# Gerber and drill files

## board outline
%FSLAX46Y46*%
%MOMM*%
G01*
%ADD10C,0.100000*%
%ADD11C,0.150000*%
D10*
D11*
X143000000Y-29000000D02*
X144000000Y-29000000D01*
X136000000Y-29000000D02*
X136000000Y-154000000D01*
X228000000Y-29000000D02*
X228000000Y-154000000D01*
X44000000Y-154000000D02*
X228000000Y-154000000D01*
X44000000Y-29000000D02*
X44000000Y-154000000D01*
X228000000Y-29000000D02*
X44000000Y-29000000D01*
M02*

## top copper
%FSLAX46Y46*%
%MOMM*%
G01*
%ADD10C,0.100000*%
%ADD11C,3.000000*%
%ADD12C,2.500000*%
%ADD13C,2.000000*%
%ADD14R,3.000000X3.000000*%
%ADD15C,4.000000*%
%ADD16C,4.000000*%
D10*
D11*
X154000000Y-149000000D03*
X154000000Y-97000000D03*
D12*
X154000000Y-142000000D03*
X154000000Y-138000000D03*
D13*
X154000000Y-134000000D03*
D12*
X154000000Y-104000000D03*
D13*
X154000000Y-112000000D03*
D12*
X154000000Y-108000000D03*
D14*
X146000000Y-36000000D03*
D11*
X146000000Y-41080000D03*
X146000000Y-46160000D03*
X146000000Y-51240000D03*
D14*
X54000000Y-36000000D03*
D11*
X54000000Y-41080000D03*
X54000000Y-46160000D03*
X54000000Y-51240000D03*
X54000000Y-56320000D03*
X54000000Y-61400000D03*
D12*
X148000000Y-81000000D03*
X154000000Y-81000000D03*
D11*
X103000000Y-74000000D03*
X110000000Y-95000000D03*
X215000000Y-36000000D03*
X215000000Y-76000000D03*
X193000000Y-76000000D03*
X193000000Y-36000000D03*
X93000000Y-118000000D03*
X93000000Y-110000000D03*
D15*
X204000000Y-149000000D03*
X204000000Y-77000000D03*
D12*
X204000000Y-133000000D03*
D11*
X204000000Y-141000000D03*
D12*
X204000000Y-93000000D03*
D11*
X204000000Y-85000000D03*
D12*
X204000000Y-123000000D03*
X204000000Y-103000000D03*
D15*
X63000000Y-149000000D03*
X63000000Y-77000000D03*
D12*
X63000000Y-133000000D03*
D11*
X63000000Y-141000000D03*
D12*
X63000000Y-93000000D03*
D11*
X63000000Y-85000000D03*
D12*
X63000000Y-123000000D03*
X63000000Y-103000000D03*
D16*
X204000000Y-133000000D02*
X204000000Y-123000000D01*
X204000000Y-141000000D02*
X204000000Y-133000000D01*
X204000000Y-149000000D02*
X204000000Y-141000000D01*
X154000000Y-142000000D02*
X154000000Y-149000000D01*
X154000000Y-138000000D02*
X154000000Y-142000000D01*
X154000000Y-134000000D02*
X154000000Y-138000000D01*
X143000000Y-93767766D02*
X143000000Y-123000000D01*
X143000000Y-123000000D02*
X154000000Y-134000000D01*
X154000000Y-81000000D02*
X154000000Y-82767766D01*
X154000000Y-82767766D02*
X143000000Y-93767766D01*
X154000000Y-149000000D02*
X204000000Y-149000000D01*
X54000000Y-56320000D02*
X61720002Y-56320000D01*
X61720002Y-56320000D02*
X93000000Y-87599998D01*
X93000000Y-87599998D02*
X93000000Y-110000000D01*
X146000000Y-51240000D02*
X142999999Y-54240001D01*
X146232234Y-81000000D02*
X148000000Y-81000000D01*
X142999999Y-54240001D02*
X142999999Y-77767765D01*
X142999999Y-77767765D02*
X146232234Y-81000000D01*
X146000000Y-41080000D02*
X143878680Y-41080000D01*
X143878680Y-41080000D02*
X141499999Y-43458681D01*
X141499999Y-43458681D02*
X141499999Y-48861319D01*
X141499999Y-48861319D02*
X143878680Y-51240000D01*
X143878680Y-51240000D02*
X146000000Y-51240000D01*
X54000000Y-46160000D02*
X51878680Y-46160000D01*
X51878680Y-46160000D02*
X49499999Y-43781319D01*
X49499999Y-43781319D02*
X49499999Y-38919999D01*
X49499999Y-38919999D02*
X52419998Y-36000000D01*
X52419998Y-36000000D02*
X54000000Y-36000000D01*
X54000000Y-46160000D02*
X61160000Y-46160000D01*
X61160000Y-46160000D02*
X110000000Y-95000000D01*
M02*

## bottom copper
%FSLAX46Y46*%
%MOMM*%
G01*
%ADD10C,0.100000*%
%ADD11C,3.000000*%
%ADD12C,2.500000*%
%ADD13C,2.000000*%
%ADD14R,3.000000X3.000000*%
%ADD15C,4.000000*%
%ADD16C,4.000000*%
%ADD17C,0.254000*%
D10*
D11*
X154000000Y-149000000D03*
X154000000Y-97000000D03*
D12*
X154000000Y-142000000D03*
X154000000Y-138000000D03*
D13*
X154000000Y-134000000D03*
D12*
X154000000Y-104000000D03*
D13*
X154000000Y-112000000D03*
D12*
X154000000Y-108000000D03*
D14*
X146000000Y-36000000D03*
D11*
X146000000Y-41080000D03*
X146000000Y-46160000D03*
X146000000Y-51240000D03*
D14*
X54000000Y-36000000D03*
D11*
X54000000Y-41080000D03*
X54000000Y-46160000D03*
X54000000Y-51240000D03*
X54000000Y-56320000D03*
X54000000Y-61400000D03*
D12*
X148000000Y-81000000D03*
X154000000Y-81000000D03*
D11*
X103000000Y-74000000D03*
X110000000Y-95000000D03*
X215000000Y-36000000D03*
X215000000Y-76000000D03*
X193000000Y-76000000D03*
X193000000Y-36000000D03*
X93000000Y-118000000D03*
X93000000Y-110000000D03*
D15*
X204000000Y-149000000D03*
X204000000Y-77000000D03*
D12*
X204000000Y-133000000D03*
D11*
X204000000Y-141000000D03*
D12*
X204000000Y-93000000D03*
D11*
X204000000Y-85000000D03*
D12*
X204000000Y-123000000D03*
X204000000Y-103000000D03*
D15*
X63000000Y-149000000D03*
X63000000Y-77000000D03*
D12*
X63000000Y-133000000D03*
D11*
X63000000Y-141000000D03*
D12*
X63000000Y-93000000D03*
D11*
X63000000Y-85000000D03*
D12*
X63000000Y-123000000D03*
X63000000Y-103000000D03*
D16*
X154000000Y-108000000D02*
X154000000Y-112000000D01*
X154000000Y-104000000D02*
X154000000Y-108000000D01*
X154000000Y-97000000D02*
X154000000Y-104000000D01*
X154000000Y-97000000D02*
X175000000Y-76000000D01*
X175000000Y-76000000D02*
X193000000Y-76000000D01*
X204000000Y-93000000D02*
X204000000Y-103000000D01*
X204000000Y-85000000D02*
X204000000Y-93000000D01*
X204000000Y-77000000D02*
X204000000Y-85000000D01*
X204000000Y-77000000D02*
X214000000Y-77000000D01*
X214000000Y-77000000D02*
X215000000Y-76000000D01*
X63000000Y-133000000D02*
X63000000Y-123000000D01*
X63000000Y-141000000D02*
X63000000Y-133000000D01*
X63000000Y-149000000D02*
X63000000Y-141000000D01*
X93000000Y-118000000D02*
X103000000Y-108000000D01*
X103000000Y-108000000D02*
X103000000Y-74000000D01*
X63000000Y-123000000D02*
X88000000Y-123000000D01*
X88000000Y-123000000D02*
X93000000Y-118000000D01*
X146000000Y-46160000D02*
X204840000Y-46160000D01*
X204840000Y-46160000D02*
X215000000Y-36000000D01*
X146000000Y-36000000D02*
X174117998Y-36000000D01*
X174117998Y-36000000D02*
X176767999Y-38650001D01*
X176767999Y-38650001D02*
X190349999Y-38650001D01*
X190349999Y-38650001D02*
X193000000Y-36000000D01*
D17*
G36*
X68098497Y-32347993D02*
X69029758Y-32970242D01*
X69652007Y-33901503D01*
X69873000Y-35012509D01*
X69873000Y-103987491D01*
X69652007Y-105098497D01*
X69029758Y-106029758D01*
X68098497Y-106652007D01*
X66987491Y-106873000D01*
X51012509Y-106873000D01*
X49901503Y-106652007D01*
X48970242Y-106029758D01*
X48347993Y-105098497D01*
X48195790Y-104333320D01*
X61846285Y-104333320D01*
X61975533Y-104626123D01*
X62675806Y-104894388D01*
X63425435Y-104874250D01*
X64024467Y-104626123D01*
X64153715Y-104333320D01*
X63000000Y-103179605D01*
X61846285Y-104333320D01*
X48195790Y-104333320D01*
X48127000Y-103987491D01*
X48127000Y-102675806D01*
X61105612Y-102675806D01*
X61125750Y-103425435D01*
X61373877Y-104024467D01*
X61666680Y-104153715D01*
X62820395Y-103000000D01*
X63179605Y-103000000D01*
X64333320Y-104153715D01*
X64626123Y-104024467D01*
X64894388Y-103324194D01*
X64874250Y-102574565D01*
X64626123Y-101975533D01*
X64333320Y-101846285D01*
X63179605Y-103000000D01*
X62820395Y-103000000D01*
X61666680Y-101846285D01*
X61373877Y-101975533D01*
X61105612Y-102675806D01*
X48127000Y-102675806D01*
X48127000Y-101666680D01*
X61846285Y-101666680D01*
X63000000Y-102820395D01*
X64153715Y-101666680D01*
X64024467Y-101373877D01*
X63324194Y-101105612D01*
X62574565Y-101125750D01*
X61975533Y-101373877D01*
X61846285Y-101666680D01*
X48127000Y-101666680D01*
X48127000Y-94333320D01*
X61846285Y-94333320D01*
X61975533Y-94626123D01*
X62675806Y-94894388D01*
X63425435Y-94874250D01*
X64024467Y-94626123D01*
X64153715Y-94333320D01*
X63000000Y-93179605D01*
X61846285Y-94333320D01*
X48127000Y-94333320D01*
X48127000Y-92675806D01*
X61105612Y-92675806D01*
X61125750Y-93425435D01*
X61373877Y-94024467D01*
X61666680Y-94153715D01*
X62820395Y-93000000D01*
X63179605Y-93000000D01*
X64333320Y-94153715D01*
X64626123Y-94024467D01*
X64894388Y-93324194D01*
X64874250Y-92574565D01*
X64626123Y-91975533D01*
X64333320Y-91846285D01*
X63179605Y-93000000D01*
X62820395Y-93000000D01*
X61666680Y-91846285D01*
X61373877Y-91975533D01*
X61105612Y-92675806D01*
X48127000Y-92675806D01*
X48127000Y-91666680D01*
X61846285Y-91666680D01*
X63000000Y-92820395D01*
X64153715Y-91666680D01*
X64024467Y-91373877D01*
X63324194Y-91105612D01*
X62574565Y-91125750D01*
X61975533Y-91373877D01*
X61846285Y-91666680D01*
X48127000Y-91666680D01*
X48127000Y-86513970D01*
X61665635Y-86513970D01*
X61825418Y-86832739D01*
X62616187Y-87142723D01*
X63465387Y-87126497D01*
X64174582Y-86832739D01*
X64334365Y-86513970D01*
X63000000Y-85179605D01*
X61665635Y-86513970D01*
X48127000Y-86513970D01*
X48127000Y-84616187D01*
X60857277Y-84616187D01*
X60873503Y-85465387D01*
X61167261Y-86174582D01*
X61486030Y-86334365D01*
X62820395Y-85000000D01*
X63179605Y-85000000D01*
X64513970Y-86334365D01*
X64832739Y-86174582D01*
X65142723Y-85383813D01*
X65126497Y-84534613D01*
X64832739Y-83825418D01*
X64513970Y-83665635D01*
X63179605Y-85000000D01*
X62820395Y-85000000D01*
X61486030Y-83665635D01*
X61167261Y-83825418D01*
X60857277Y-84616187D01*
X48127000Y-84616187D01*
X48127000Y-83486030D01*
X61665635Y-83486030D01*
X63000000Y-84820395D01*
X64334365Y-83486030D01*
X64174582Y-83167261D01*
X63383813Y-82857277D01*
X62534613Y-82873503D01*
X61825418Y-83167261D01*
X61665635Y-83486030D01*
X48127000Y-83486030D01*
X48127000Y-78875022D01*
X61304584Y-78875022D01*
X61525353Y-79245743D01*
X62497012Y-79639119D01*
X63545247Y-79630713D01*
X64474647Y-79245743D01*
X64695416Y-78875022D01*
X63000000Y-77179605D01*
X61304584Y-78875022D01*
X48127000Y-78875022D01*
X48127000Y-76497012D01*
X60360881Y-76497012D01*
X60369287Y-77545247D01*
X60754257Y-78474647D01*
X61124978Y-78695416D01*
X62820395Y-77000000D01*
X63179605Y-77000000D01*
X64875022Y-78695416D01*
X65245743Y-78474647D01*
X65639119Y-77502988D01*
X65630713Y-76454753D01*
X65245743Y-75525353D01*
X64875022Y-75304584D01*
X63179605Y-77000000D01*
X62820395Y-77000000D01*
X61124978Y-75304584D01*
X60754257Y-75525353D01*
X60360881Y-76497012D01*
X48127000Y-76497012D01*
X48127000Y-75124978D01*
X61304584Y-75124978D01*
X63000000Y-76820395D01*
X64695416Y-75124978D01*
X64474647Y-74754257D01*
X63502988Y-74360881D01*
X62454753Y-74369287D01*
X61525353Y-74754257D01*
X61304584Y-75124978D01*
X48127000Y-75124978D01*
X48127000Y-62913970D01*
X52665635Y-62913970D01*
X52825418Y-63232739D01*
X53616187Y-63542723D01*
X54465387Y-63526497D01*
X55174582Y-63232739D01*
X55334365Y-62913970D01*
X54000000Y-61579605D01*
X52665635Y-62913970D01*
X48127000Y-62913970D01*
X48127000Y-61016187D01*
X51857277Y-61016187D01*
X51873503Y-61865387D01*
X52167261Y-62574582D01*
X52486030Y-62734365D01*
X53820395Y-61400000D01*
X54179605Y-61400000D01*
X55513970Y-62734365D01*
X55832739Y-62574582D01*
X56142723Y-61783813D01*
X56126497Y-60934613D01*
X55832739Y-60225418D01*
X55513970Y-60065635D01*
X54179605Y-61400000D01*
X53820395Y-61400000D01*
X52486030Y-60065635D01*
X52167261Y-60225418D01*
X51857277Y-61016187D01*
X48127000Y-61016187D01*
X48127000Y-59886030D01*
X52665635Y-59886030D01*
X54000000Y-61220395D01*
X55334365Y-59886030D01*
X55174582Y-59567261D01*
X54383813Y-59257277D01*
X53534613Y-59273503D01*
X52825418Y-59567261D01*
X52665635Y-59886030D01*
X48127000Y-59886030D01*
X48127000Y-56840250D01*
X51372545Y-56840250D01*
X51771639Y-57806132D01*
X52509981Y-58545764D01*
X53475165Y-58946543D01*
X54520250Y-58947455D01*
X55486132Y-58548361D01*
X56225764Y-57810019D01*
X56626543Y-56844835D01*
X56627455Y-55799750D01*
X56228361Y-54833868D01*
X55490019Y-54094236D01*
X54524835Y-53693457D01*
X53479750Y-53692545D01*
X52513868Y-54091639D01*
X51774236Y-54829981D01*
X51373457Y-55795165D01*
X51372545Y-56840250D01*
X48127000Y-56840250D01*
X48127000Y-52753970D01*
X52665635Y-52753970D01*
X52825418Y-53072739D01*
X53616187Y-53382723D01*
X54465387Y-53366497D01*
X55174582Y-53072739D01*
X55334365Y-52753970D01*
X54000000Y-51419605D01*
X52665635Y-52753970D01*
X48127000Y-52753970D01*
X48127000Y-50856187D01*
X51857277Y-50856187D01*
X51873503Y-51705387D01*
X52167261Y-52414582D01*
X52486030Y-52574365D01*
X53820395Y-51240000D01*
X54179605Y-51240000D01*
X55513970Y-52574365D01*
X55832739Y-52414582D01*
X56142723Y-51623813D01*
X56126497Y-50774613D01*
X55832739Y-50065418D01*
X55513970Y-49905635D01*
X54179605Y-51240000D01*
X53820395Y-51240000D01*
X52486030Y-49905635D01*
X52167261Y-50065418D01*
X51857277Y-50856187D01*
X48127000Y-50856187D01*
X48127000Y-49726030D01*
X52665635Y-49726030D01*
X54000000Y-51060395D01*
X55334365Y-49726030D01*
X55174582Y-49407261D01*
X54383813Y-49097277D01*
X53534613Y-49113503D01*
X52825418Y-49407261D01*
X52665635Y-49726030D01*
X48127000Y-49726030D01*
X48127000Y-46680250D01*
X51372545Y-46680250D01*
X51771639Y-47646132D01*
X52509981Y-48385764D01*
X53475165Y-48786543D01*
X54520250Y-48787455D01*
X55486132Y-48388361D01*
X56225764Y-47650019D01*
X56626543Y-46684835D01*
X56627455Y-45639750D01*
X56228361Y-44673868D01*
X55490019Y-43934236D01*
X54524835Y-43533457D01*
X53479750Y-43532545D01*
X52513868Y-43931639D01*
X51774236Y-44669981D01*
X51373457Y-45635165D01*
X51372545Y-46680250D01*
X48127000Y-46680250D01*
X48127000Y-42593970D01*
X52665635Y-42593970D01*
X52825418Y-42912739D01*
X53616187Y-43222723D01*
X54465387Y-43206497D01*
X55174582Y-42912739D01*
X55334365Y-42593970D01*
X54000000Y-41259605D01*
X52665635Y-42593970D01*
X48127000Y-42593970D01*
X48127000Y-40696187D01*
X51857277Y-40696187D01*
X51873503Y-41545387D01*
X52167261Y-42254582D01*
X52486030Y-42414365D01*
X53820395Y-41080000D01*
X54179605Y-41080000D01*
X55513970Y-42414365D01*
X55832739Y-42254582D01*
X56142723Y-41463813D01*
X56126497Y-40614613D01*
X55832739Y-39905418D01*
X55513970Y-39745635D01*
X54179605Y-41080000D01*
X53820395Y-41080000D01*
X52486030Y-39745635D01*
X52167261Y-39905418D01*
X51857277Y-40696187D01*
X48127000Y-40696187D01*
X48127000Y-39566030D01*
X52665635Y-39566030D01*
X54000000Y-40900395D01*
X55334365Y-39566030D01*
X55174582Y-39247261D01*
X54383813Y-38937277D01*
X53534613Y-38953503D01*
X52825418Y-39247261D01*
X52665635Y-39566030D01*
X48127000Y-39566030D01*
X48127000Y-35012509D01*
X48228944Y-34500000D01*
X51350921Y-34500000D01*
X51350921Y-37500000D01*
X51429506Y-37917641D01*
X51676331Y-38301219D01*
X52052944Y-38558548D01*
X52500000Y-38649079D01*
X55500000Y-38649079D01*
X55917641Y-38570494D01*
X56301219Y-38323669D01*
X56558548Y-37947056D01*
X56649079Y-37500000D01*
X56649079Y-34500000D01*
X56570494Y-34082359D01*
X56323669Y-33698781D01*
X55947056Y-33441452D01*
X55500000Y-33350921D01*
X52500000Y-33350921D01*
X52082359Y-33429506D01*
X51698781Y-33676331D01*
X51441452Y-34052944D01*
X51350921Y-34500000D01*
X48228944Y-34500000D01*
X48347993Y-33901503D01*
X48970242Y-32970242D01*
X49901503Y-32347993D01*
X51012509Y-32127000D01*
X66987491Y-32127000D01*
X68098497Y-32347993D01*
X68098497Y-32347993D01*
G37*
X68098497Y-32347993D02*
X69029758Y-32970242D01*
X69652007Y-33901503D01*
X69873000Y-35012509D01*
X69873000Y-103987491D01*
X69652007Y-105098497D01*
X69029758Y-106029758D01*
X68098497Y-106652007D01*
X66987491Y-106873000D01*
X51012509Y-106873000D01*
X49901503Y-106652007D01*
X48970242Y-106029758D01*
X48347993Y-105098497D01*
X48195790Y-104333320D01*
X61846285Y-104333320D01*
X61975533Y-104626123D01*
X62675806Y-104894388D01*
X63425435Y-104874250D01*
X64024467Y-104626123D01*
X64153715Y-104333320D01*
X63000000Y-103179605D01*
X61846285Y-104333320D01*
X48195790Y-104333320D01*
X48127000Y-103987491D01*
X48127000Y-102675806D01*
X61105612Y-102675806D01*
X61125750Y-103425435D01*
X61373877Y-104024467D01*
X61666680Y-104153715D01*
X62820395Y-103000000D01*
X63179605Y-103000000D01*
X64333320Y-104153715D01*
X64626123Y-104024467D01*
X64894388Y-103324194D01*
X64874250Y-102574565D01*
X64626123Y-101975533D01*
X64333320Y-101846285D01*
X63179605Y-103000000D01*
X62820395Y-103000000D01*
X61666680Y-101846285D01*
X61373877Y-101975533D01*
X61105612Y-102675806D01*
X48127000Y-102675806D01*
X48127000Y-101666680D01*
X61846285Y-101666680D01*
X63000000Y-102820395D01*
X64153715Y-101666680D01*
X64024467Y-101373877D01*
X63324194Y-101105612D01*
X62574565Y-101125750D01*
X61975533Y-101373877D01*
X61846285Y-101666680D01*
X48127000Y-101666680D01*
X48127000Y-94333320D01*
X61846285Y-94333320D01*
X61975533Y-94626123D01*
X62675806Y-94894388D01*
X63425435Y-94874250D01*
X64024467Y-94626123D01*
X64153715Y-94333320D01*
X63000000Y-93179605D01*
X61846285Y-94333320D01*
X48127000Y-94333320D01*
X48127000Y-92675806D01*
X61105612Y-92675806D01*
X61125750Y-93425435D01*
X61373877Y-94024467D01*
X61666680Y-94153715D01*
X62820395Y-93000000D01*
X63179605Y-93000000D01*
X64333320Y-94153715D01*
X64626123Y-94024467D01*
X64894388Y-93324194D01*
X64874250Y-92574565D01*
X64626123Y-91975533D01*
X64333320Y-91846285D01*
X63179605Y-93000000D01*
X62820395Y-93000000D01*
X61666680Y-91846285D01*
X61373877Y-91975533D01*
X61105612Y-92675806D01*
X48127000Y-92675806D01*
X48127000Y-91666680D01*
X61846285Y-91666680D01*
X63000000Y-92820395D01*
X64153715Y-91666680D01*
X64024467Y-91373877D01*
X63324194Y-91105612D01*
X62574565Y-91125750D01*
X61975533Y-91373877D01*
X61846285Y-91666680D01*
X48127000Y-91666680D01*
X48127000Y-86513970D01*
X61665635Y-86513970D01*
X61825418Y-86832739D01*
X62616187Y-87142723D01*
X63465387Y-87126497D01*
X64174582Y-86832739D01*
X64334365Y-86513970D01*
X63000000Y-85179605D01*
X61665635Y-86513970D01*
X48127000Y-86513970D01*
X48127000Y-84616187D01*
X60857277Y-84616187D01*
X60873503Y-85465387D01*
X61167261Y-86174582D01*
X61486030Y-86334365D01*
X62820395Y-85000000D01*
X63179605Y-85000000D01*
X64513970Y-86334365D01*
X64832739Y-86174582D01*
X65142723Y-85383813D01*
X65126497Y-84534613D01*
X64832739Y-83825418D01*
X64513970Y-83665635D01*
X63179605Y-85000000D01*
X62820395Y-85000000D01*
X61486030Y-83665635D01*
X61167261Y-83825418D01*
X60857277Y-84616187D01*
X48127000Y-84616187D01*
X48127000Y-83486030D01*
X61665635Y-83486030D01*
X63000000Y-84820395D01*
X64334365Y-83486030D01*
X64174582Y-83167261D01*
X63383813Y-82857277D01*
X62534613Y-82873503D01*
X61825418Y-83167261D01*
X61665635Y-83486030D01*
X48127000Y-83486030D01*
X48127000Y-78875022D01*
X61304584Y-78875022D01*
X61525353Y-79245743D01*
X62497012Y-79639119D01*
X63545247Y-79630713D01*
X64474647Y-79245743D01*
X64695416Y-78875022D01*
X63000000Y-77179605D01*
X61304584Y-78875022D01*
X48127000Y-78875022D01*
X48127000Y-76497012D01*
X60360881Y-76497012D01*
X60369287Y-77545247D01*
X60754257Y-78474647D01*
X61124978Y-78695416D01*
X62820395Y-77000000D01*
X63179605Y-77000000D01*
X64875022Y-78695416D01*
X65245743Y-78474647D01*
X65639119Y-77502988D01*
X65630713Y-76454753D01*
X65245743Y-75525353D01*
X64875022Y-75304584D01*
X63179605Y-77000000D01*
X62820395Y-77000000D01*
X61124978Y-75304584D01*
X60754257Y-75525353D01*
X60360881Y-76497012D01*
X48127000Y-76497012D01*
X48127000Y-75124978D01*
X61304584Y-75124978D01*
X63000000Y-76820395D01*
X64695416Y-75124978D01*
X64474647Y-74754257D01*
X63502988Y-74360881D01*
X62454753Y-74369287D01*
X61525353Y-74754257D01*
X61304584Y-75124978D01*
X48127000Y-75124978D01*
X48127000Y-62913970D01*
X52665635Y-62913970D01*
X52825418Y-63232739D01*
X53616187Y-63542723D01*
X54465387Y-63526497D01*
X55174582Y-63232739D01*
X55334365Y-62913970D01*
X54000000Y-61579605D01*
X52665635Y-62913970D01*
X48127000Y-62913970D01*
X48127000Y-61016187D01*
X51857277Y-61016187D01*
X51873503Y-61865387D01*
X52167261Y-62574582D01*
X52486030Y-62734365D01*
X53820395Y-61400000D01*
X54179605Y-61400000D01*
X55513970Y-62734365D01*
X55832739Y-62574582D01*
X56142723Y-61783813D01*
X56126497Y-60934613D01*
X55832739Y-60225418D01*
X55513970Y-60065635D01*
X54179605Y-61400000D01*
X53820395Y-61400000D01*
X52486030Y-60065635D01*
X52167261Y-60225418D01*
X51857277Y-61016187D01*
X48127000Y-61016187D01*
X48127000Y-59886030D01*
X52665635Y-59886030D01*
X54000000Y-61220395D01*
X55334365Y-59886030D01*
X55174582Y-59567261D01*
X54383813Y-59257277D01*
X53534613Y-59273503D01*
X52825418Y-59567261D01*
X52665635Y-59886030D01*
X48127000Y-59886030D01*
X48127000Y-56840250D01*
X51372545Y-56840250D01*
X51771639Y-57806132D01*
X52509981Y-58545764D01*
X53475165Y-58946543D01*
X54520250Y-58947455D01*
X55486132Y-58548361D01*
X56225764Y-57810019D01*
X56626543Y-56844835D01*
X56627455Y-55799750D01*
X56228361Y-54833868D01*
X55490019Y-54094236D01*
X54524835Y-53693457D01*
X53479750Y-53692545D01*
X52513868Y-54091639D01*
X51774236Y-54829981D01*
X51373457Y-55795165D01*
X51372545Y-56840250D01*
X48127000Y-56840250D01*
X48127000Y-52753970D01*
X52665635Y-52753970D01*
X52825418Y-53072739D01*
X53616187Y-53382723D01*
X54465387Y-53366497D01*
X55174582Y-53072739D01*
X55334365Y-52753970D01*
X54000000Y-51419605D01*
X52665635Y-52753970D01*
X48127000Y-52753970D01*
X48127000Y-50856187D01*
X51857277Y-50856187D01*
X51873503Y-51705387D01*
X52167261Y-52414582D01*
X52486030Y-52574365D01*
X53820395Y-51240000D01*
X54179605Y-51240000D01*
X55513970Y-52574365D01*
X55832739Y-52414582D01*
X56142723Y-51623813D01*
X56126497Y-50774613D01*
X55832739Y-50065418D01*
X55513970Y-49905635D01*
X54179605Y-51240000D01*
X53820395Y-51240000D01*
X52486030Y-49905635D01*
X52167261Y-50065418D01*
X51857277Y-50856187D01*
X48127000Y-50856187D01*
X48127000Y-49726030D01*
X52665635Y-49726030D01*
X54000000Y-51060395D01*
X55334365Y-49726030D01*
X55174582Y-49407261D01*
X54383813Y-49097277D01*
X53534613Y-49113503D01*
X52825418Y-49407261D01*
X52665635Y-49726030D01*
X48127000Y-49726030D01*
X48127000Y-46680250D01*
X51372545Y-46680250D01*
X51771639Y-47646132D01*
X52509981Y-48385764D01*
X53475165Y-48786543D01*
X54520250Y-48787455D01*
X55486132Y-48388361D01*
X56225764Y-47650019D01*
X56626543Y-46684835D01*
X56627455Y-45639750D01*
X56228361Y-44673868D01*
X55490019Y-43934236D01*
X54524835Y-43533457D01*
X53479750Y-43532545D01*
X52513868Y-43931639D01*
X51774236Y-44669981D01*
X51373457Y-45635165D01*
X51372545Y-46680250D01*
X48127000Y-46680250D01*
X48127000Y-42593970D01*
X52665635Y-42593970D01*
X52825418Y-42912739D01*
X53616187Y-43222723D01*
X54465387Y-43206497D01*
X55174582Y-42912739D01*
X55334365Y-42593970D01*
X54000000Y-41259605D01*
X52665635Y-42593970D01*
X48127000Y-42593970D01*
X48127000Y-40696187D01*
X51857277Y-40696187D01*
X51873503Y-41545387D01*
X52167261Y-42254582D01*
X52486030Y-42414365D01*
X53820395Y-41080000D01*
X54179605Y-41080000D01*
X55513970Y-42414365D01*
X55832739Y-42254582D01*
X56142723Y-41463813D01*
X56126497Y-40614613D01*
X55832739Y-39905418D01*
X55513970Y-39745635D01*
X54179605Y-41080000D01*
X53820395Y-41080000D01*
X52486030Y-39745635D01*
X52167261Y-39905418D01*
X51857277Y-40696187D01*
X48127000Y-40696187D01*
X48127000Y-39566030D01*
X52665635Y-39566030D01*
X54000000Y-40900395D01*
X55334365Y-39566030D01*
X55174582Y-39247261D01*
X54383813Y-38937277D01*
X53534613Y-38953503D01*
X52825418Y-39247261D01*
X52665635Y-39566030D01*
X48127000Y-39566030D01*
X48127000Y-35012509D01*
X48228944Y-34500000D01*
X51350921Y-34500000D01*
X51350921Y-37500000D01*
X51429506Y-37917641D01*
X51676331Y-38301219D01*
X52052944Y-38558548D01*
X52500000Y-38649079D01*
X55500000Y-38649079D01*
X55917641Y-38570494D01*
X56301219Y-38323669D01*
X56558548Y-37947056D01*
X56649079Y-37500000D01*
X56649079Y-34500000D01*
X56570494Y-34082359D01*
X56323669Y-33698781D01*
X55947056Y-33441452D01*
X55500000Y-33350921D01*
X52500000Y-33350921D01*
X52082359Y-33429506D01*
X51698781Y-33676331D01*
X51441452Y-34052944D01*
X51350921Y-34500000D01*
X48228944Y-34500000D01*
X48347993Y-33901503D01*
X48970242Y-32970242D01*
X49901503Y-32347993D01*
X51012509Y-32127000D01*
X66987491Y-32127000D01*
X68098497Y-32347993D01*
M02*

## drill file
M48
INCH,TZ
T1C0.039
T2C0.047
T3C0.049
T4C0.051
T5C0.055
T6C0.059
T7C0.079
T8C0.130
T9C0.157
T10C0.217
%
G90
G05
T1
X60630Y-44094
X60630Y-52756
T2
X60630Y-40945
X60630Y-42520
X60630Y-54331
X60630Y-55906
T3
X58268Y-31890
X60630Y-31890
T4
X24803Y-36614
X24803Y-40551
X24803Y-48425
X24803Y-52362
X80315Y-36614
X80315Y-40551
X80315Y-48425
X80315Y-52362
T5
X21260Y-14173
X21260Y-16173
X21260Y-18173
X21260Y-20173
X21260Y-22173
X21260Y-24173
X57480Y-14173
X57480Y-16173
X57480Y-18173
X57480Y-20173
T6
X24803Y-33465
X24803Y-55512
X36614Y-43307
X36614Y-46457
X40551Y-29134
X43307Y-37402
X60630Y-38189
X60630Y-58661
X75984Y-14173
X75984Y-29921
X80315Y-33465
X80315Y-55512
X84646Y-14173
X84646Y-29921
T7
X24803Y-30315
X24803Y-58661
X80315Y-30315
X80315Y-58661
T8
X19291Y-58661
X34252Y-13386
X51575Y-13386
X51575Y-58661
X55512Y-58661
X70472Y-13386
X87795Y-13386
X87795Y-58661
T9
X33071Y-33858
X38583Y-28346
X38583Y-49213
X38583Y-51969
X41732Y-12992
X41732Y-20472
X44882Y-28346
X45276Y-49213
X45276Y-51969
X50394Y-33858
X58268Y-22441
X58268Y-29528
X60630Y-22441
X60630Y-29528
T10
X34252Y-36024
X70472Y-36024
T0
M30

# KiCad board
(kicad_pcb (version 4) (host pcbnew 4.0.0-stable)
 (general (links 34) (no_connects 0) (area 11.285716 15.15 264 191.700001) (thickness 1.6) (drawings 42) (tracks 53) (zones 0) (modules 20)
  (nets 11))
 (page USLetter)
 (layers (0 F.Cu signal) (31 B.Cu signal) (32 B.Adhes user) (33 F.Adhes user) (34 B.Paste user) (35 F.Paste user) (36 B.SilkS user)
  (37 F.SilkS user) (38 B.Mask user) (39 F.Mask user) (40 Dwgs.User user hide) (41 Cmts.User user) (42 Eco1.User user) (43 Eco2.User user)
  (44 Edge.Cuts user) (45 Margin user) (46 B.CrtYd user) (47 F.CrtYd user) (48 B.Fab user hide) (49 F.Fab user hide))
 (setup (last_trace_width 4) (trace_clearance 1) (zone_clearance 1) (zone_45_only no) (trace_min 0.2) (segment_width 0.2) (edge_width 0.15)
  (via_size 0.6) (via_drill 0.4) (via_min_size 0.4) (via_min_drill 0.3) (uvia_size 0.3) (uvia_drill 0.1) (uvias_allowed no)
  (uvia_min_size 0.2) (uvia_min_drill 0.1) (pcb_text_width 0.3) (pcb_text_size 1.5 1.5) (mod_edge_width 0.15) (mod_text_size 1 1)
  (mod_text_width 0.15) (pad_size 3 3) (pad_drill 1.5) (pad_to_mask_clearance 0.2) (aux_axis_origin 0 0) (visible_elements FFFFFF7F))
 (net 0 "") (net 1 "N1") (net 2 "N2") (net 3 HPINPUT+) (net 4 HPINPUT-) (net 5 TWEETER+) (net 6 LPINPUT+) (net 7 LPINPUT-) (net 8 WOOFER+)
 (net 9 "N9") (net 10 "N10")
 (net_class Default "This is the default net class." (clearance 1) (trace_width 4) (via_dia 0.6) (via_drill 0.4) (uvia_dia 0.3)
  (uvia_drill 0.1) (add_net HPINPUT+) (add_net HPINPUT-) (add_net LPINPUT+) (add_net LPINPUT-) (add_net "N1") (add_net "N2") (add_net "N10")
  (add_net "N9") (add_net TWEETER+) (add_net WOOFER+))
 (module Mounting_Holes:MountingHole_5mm (layer F.Cu) (at 179 91.5)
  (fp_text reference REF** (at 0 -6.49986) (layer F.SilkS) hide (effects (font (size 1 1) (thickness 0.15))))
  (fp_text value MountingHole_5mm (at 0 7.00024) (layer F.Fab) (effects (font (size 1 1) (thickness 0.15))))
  (pad "" np_thru_hole circle (at 0 0) (size 5.5 5.5) (drill 5.5) (layers *.Cu *.Mask F.SilkS)))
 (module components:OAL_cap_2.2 (layer F.Cu) (at 154 123 90)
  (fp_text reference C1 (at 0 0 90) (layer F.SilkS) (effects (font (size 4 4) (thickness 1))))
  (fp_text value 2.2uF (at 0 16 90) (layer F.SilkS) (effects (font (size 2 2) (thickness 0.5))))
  (pad 1 thru_hole circle (at -26 0 90) (size 3 3) (drill 1.5) (layers *.Cu *.Mask F.SilkS) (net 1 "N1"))
  (pad 2 thru_hole circle (at 26 0 90) (size 3 3) (drill 1.5) (layers *.Cu *.Mask F.SilkS) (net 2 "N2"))
  (pad 1 thru_hole circle (at -19 0 90) (size 2.5 2.5) (drill 1.2) (layers *.Cu *.Mask F.SilkS) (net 1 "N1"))
  (pad 1 thru_hole circle (at -15 0 90) (size 2.5 2.5) (drill 1.2) (layers *.Cu *.Mask F.SilkS) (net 1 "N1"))
  (pad 1 thru_hole circle (at -11 0 90) (size 2 2) (drill 1) (layers *.Cu *.Mask F.SilkS) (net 1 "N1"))
  (pad 2 thru_hole circle (at 19 0 270) (size 2.5 2.5) (drill 1.2) (layers *.Cu *.Mask F.SilkS) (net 2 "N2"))
  (pad 2 thru_hole circle (at 11 0 270) (size 2 2) (drill 1) (layers *.Cu *.Mask F.SilkS) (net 2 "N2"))
  (pad 2 thru_hole circle (at 15 0 270) (size 2.5 2.5) (drill 1.2) (layers *.Cu *.Mask F.SilkS) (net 2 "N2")))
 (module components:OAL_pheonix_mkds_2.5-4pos (layer F.Cu) (at 146 36 270)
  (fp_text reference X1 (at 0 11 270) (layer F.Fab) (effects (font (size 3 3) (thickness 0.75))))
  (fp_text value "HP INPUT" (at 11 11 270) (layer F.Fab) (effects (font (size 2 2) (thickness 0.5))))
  (pad 1 thru_hole rect (at 0 0 270) (size 3 3) (drill 1.4) (layers *.Cu *.Mask F.SilkS) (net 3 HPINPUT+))
  (pad 2 thru_hole circle (at 5.08 0 270) (size 3 3) (drill 1.4) (layers *.Cu *.Mask F.SilkS) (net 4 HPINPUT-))
  (pad 3 thru_hole circle (at 10.16 0 270) (size 3 3) (drill 1.4) (layers *.Cu *.Mask F.SilkS) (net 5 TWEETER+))
  (pad 4 thru_hole circle (at 15.24 0 270) (size 3 3) (drill 1.4) (layers *.Cu *.Mask F.SilkS) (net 4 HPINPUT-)))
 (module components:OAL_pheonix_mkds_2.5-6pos (layer F.Cu) (at 54 36 270)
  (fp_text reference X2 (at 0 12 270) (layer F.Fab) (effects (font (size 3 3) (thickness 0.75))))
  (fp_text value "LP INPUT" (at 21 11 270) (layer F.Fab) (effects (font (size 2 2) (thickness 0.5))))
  (pad 1 thru_hole rect (at 0 0 270) (size 3 3) (drill 1.4) (layers *.Cu *.Mask F.SilkS) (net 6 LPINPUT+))
  (pad 2 thru_hole circle (at 5.08 0 270) (size 3 3) (drill 1.4) (layers *.Cu *.Mask F.SilkS) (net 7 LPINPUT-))
  (pad 3 thru_hole circle (at 10.16 0 270) (size 3 3) (drill 1.4) (layers *.Cu *.Mask F.SilkS) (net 6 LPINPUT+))
  (pad 4 thru_hole circle (at 15.24 0 270) (size 3 3) (drill 1.4) (layers *.Cu *.Mask F.SilkS) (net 7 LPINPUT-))
  (pad 5 thru_hole circle (at 20.32 0 270) (size 3 3) (drill 1.4) (layers *.Cu *.Mask F.SilkS) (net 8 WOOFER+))
  (pad 6 thru_hole circle (at 25.4 0 270) (size 3 3) (drill 1.4) (layers *.Cu *.Mask F.SilkS) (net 7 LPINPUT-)))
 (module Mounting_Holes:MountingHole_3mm (layer F.Cu) (at 87 34)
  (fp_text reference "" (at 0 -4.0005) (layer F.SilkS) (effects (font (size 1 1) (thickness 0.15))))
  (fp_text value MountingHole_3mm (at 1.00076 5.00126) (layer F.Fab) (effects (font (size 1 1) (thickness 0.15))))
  (pad "" np_thru_hole circle (at 0 0) (size 3.3 3.3) (drill 3.3) (layers *.Cu *.Mask F.SilkS)))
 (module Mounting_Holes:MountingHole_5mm (layer F.Cu) (at 87 91.5)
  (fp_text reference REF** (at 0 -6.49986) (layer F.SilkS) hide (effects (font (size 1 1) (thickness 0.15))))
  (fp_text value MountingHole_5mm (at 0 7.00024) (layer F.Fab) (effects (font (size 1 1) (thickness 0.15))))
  (pad "" np_thru_hole circle (at 0 0) (size 5.5 5.5) (drill 5.5) (layers *.Cu *.Mask F.SilkS)))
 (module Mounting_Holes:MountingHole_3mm (layer F.Cu) (at 179 34)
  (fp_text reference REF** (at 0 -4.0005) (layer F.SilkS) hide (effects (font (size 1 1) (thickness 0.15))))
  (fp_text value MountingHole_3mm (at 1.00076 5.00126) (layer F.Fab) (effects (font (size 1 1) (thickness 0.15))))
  (pad "" np_thru_hole circle (at 0 0) (size 3.3 3.3) (drill 3.3) (layers *.Cu *.Mask F.SilkS)))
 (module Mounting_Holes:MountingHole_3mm (layer F.Cu) (at 141 149)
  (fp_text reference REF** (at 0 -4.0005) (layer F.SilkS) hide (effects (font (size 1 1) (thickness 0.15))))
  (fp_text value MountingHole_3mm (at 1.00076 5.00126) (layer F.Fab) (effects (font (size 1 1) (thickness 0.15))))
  (pad "" np_thru_hole circle (at 0 0) (size 3.3 3.3) (drill 3.3) (layers *.Cu *.Mask F.SilkS)))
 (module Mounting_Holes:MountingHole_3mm (layer F.Cu) (at 223 149)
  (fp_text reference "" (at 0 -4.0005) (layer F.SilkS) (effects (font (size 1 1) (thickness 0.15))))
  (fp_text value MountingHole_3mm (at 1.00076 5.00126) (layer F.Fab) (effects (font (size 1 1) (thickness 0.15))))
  (pad "" np_thru_hole circle (at 0 0) (size 3.3 3.3) (drill 3.3) (layers *.Cu *.Mask F.SilkS)))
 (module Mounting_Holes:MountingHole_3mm (layer F.Cu) (at 131 34)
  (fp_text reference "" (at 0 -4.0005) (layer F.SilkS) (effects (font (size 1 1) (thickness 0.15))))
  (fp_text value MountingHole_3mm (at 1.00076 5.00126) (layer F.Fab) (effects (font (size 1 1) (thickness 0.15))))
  (pad "" np_thru_hole circle (at 0 0) (size 3.3 3.3) (drill 3.3) (layers *.Cu *.Mask F.SilkS)))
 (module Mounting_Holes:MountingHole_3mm (layer F.Cu) (at 49 149)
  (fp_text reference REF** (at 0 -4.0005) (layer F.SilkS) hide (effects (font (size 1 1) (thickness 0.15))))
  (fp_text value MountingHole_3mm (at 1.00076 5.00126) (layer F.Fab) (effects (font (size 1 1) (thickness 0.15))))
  (pad "" np_thru_hole circle (at 0 0) (size 3.3 3.3) (drill 3.3) (layers *.Cu *.Mask F.SilkS)))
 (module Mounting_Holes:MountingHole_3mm (layer F.Cu) (at 223 34)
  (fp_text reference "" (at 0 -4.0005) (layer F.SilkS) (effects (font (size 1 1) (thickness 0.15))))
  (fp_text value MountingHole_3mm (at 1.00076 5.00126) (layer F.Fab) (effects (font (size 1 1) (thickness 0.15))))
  (pad "" np_thru_hole circle (at 0 0) (size 3.3 3.3) (drill 3.3) (layers *.Cu *.Mask F.SilkS)))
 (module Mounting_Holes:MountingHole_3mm (layer F.Cu) (at 131 149)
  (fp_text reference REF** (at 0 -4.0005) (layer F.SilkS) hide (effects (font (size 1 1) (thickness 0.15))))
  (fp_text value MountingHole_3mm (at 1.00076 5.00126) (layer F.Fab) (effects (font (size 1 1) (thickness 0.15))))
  (pad "" np_thru_hole circle (at 0 0) (size 3.3 3.3) (drill 3.3) (layers *.Cu *.Mask F.SilkS)))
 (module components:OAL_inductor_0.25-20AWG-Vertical (layer F.Cu) (at 151 66 180)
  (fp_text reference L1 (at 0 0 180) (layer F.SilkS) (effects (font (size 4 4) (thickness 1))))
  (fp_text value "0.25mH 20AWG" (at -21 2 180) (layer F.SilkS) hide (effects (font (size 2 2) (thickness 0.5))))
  (pad "" np_thru_hole circle (at -3 -9 180) (size 4 4) (drill 4) (layers *.Cu *.Mask F.SilkS))
  (pad "" np_thru_hole circle (at 3 9 180) (size 4 4) (drill 4) (layers *.Cu *.Mask F.SilkS))
  (pad "" np_thru_hole circle (at 3 -9 180) (size 4 4) (drill 4) (layers *.Cu *.Mask F.SilkS))
  (pad 2 thru_hole circle (at 3 -15 180) (size 2.5 2.5) (drill 1.25) (layers *.Cu *.Mask F.SilkS) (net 4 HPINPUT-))
  (pad 1 thru_hole circle (at -3 -15 180) (size 2.5 2.5) (drill 1.25) (layers *.Cu *.Mask F.SilkS) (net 1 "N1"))
  (pad "" np_thru_hole circle (at -3 9 180) (size 4 4) (drill 4) (layers *.Cu *.Mask F.SilkS)))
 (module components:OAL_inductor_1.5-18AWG (layer F.Cu) (at 106 64 180)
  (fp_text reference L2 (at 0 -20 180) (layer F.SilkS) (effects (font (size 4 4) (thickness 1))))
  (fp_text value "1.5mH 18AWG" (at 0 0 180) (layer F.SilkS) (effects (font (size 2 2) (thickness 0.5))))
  (pad "" np_thru_hole circle (at -8 -8 180) (size 4 4) (drill 4) (layers *.Cu *.Mask F.SilkS))
  (pad "" np_thru_hole circle (at -22 -22 180) (size 4 4) (drill 4) (layers *.Cu *.Mask F.SilkS))
  (pad "" np_thru_hole circle (at 22 -22 180) (size 4 4) (drill 4) (layers *.Cu *.Mask F.SilkS))
  (pad "" np_thru_hole circle (at 8 -8 180) (size 4 4) (drill 4) (layers *.Cu *.Mask F.SilkS))
  (pad "" np_thru_hole circle (at 0 31 180) (size 4 4) (drill 4) (layers *.Cu *.Mask F.SilkS))
  (pad 1 thru_hole circle (at 3 -10 180) (size 3 3) (drill 1.5) (layers *.Cu *.Mask F.SilkS) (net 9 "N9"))
  (pad 2 thru_hole circle (at -4 -31 180) (size 3 3) (drill 1.5) (layers *.Cu *.Mask F.SilkS) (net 6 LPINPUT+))
  (pad "" np_thru_hole circle (at 0 12 180) (size 4 4) (drill 4) (layers *.Cu *.Mask F.SilkS)))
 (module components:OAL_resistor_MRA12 (layer F.Cu) (at 215 56 270)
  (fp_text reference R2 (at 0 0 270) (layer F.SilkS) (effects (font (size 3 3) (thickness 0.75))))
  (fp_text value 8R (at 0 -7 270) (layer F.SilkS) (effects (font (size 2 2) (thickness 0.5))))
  (pad 1 thru_hole circle (at -20 0 270) (size 3 3) (drill 1.5) (layers *.Cu *.Mask F.SilkS) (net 5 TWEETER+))
  (pad 2 thru_hole circle (at 20 0 270) (size 3 3) (drill 1.5) (layers *.Cu *.Mask F.SilkS) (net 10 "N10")))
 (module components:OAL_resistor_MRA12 (layer F.Cu) (at 193 56 90)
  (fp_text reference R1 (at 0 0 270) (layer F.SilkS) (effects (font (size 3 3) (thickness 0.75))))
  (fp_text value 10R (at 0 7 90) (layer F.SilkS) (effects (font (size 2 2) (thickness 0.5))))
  (pad 1 thru_hole circle (at -20 0 90) (size 3 3) (drill 1.5) (layers *.Cu *.Mask F.SilkS) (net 2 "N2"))
  (pad 2 thru_hole circle (at 20 0 90) (size 3 3) (drill 1.5) (layers *.Cu *.Mask F.SilkS) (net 3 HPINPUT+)))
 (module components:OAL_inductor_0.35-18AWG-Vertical (layer F.Cu) (at 99 106 270)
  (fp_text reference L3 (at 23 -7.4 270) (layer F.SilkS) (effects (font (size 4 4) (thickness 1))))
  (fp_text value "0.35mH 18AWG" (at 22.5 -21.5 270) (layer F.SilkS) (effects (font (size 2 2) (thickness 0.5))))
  (pad "" np_thru_hole circle (at 19 -16 270) (size 4 4) (drill 4) (layers *.Cu *.Mask F.SilkS))
  (pad "" np_thru_hole circle (at 26 -16 270) (size 4 4) (drill 4) (layers *.Cu *.Mask F.SilkS))
  (pad 2 thru_hole circle (at 12 6 270) (size 3 3) (drill 1.5) (layers *.Cu *.Mask F.SilkS) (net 9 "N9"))
  (pad 1 thru_hole circle (at 4 6 270) (size 3 3) (drill 1.5) (layers *.Cu *.Mask F.SilkS) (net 8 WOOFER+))
  (pad "" np_thru_hole circle (at 19 1 270) (size 4 4) (drill 4) (layers *.Cu *.Mask F.SilkS))
  (pad "" np_thru_hole circle (at 26 1 270) (size 4 4) (drill 4) (layers *.Cu *.Mask F.SilkS)))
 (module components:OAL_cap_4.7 (layer F.Cu) (at 204 113 90)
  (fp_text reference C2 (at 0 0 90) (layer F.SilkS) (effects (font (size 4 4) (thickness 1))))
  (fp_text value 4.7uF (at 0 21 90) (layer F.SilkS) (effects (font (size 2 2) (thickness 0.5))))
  (pad 1 thru_hole circle (at -36 0 90) (size 4 4) (drill 2) (layers *.Cu *.Mask F.SilkS) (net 1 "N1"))
  (pad 2 thru_hole circle (at 36 0 90) (size 4 4) (drill 2) (layers *.Cu *.Mask F.SilkS) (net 10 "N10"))
  (pad 1 thru_hole circle (at -20 0 90) (size 2.5 2.5) (drill 1.3) (layers *.Cu *.Mask F.SilkS) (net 1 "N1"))
  (pad 1 thru_hole circle (at -28 0 90) (size 3 3) (drill 1.5) (layers *.Cu *.Mask F.SilkS) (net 1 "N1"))
  (pad 2 thru_hole circle (at 20 0 90) (size 2.5 2.5) (drill 1.3) (layers *.Cu *.Mask F.SilkS) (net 10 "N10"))
  (pad 2 thru_hole circle (at 28 0 90) (size 3 3) (drill 1.5) (layers *.Cu *.Mask F.SilkS) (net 10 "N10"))
  (pad 1 thru_hole circle (at -10 0 90) (size 2.5 2.5) (drill 1.3) (layers *.Cu *.Mask F.SilkS) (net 1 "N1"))
  (pad 2 thru_hole circle (at 10 0 90) (size 2.5 2.5) (drill 1.3) (layers *.Cu *.Mask F.SilkS) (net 10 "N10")))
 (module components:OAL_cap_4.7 (layer F.Cu) (at 63 113 90)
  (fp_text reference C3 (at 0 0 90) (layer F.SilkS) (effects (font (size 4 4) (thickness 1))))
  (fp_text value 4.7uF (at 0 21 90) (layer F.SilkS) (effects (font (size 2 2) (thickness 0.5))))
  (pad 1 thru_hole circle (at -36 0 90) (size 4 4) (drill 2) (layers *.Cu *.Mask F.SilkS) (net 9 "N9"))
  (pad 2 thru_hole circle (at 36 0 90) (size 4 4) (drill 2) (layers *.Cu *.Mask F.SilkS) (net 7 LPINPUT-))
  (pad 1 thru_hole circle (at -20 0 90) (size 2.5 2.5) (drill 1.3) (layers *.Cu *.Mask F.SilkS) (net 9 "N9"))
  (pad 1 thru_hole circle (at -28 0 90) (size 3 3) (drill 1.5) (layers *.Cu *.Mask F.SilkS) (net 9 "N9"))
  (pad 2 thru_hole circle (at 20 0 90) (size 2.5 2.5) (drill 1.3) (layers *.Cu *.Mask F.SilkS) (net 7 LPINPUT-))
  (pad 2 thru_hole circle (at 28 0 90) (size 3 3) (drill 1.5) (layers *.Cu *.Mask F.SilkS) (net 7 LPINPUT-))
  (pad 1 thru_hole circle (at -10 0 90) (size 2.5 2.5) (drill 1.3) (layers *.Cu *.Mask F.SilkS) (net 9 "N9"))
  (pad 2 thru_hole circle (at 10 0 90) (size 2.5 2.5) (drill 1.3) (layers *.Cu *.Mask F.SilkS) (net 7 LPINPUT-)))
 (gr_line (start 143 29) (end 144 29) (layer Edge.Cuts) (width 0.15))
 (gr_line (start 136 29) (end 136 154) (layer Edge.Cuts) (width 0.15))
 (gr_line (start 228 29) (end 228 154) (layer Edge.Cuts) (width 0.15))
 (gr_line (start 44 154) (end 228 154) (layer Edge.Cuts) (width 0.15))
 (gr_line (start 44 29) (end 44 154) (layer Edge.Cuts) (width 0.15))
 (gr_line (start 228 29) (end 44 29) (layer Edge.Cuts) (width 0.15))
 (segment (start 204 133) (end 204 123) (width 4) (layer F.Cu) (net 1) (status 30))
 (segment (start 204 141) (end 204 133) (width 4) (layer F.Cu) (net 1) (status 30))
 (segment (start 204 149) (end 204 141) (width 4) (layer F.Cu) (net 1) (status 30))
 (segment (start 154 142) (end 154 149) (width 4) (layer F.Cu) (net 1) (status 30))
 (segment (start 154 138) (end 154 142) (width 4) (layer F.Cu) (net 1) (status 30))
 (segment (start 154 134) (end 154 138) (width 4) (layer F.Cu) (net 1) (status 30))
 (segment (start 143 93.767766) (end 143 123) (width 4) (layer F.Cu) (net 1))
 (segment (start 143 123) (end 154 134) (width 4) (layer F.Cu) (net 1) (status 20))
 (segment (start 154 81) (end 154 82.767766) (width 4) (layer F.Cu) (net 1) (status 10))
 (segment (start 154 82.767766) (end 143 93.767766) (width 4) (layer F.Cu) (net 1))
 (segment (start 154 149) (end 204 149) (width 4) (layer F.Cu) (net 1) (status 30))
 (segment (start 154 108) (end 154 112) (width 4) (layer B.Cu) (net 2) (status 30))
 (segment (start 154 104) (end 154 108) (width 4) (layer B.Cu) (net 2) (status 30))
 (segment (start 154 97) (end 154 104) (width 4) (layer B.Cu) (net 2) (status 30))
 (segment (start 154 97) (end 175 76) (width 4) (layer B.Cu) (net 2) (status 10))
 (segment (start 175 76) (end 193 76) (width 4) (layer B.Cu) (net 2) (status 20))
 (segment (start 204 93) (end 204 103) (width 4) (layer B.Cu) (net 10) (status 30))
 (segment (start 204 85) (end 204 93) (width 4) (layer B.Cu) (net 10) (status 30))
 (segment (start 204 77) (end 204 85) (width 4) (layer B.Cu) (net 10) (status 30))
 (segment (start 204 77) (end 214 77) (width 4) (layer B.Cu) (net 10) (status 30))
 (segment (start 214 77) (end 215 76) (width 4) (layer B.Cu) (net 10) (status 30))
 (segment (start 63 133) (end 63 123) (width 4) (layer B.Cu) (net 9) (status 30))
 (segment (start 63 141) (end 63 133) (width 4) (layer B.Cu) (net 9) (status 30))
 (segment (start 63 149) (end 63 141) (width 4) (layer B.Cu) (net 9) (status 30))
 (segment (start 93 118) (end 103 108) (width 4) (layer B.Cu) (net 9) (status 10))
 (segment (start 103 108) (end 103 74) (width 4) (layer B.Cu) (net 9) (status 20))
 (segment (start 63 123) (end 88 123) (width 4) (layer B.Cu) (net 9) (status 10))
 (segment (start 88 123) (end 93 118) (width 4) (layer B.Cu) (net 9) (status 20))
 (segment (start 54 56.32) (end 61.720002 56.32) (width 4) (layer F.Cu) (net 8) (status 10))
 (segment (start 61.720002 56.32) (end 93 87.599998) (width 4) (layer F.Cu) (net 8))
 (segment (start 93 87.599998) (end 93 110) (width 4) (layer F.Cu) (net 8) (status 20))
 (segment (start 146 46.16) (end 204.84 46.16) (width 4) (layer B.Cu) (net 5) (status 10))
 (segment (start 204.84 46.16) (end 215 36) (width 4) (layer B.Cu) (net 5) (status 20))
 (segment (start 146 51.24) (end 142.999999 54.240001) (width 4) (layer F.Cu) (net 4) (status 10))
 (segment (start 146.232234 81) (end 148 81) (width 4) (layer F.Cu) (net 4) (status 20))
 (segment (start 142.999999 54.240001) (end 142.999999 77.767765) (width 4) (layer F.Cu) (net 4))
 (segment (start 142.999999 77.767765) (end 146.232234 81) (width 4) (layer F.Cu) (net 4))
 (segment (start 146 41.08) (end 143.87868 41.08) (width 4) (layer F.Cu) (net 4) (status 10))
 (segment (start 143.87868 41.08) (end 141.499999 43.458681) (width 4) (layer F.Cu) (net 4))
 (segment (start 141.499999 43.458681) (end 141.499999 48.861319) (width 4) (layer F.Cu) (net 4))
 (segment (start 141.499999 48.861319) (end 143.87868 51.24) (width 4) (layer F.Cu) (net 4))
 (segment (start 143.87868 51.24) (end 146 51.24) (width 4) (layer F.Cu) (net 4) (status 20))
 (segment (start 54 46.16) (end 51.87868 46.16) (width 4) (layer F.Cu) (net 6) (status 10))
 (segment (start 51.87868 46.16) (end 49.499999 43.781319) (width 4) (layer F.Cu) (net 6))
 (segment (start 49.499999 43.781319) (end 49.499999 38.919999) (width 4) (layer F.Cu) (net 6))
 (segment (start 49.499999 38.919999) (end 52.419998 36) (width 4) (layer F.Cu) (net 6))
 (segment (start 52.419998 36) (end 54 36) (width 4) (layer F.Cu) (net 6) (status 20))
 (segment (start 54 46.16) (end 61.16 46.16) (width 4) (layer F.Cu) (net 6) (status 10))
 (segment (start 61.16 46.16) (end 110 95) (width 4) (layer F.Cu) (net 6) (status 20))
 (segment (start 146 36) (end 174.117998 36) (width 4) (layer B.Cu) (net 3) (status 10))
 (segment (start 174.117998 36) (end 176.767999 38.650001) (width 4) (layer B.Cu) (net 3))
 (segment (start 176.767999 38.650001) (end 190.349999 38.650001) (width 4) (layer B.Cu) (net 3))
 (segment (start 190.349999 38.650001) (end 193 36) (width 4) (layer B.Cu) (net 3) (status 20))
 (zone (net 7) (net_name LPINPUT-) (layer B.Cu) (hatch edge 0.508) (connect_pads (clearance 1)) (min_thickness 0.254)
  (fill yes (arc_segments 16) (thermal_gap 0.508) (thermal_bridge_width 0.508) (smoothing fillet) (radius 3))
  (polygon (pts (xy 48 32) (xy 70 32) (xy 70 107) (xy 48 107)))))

